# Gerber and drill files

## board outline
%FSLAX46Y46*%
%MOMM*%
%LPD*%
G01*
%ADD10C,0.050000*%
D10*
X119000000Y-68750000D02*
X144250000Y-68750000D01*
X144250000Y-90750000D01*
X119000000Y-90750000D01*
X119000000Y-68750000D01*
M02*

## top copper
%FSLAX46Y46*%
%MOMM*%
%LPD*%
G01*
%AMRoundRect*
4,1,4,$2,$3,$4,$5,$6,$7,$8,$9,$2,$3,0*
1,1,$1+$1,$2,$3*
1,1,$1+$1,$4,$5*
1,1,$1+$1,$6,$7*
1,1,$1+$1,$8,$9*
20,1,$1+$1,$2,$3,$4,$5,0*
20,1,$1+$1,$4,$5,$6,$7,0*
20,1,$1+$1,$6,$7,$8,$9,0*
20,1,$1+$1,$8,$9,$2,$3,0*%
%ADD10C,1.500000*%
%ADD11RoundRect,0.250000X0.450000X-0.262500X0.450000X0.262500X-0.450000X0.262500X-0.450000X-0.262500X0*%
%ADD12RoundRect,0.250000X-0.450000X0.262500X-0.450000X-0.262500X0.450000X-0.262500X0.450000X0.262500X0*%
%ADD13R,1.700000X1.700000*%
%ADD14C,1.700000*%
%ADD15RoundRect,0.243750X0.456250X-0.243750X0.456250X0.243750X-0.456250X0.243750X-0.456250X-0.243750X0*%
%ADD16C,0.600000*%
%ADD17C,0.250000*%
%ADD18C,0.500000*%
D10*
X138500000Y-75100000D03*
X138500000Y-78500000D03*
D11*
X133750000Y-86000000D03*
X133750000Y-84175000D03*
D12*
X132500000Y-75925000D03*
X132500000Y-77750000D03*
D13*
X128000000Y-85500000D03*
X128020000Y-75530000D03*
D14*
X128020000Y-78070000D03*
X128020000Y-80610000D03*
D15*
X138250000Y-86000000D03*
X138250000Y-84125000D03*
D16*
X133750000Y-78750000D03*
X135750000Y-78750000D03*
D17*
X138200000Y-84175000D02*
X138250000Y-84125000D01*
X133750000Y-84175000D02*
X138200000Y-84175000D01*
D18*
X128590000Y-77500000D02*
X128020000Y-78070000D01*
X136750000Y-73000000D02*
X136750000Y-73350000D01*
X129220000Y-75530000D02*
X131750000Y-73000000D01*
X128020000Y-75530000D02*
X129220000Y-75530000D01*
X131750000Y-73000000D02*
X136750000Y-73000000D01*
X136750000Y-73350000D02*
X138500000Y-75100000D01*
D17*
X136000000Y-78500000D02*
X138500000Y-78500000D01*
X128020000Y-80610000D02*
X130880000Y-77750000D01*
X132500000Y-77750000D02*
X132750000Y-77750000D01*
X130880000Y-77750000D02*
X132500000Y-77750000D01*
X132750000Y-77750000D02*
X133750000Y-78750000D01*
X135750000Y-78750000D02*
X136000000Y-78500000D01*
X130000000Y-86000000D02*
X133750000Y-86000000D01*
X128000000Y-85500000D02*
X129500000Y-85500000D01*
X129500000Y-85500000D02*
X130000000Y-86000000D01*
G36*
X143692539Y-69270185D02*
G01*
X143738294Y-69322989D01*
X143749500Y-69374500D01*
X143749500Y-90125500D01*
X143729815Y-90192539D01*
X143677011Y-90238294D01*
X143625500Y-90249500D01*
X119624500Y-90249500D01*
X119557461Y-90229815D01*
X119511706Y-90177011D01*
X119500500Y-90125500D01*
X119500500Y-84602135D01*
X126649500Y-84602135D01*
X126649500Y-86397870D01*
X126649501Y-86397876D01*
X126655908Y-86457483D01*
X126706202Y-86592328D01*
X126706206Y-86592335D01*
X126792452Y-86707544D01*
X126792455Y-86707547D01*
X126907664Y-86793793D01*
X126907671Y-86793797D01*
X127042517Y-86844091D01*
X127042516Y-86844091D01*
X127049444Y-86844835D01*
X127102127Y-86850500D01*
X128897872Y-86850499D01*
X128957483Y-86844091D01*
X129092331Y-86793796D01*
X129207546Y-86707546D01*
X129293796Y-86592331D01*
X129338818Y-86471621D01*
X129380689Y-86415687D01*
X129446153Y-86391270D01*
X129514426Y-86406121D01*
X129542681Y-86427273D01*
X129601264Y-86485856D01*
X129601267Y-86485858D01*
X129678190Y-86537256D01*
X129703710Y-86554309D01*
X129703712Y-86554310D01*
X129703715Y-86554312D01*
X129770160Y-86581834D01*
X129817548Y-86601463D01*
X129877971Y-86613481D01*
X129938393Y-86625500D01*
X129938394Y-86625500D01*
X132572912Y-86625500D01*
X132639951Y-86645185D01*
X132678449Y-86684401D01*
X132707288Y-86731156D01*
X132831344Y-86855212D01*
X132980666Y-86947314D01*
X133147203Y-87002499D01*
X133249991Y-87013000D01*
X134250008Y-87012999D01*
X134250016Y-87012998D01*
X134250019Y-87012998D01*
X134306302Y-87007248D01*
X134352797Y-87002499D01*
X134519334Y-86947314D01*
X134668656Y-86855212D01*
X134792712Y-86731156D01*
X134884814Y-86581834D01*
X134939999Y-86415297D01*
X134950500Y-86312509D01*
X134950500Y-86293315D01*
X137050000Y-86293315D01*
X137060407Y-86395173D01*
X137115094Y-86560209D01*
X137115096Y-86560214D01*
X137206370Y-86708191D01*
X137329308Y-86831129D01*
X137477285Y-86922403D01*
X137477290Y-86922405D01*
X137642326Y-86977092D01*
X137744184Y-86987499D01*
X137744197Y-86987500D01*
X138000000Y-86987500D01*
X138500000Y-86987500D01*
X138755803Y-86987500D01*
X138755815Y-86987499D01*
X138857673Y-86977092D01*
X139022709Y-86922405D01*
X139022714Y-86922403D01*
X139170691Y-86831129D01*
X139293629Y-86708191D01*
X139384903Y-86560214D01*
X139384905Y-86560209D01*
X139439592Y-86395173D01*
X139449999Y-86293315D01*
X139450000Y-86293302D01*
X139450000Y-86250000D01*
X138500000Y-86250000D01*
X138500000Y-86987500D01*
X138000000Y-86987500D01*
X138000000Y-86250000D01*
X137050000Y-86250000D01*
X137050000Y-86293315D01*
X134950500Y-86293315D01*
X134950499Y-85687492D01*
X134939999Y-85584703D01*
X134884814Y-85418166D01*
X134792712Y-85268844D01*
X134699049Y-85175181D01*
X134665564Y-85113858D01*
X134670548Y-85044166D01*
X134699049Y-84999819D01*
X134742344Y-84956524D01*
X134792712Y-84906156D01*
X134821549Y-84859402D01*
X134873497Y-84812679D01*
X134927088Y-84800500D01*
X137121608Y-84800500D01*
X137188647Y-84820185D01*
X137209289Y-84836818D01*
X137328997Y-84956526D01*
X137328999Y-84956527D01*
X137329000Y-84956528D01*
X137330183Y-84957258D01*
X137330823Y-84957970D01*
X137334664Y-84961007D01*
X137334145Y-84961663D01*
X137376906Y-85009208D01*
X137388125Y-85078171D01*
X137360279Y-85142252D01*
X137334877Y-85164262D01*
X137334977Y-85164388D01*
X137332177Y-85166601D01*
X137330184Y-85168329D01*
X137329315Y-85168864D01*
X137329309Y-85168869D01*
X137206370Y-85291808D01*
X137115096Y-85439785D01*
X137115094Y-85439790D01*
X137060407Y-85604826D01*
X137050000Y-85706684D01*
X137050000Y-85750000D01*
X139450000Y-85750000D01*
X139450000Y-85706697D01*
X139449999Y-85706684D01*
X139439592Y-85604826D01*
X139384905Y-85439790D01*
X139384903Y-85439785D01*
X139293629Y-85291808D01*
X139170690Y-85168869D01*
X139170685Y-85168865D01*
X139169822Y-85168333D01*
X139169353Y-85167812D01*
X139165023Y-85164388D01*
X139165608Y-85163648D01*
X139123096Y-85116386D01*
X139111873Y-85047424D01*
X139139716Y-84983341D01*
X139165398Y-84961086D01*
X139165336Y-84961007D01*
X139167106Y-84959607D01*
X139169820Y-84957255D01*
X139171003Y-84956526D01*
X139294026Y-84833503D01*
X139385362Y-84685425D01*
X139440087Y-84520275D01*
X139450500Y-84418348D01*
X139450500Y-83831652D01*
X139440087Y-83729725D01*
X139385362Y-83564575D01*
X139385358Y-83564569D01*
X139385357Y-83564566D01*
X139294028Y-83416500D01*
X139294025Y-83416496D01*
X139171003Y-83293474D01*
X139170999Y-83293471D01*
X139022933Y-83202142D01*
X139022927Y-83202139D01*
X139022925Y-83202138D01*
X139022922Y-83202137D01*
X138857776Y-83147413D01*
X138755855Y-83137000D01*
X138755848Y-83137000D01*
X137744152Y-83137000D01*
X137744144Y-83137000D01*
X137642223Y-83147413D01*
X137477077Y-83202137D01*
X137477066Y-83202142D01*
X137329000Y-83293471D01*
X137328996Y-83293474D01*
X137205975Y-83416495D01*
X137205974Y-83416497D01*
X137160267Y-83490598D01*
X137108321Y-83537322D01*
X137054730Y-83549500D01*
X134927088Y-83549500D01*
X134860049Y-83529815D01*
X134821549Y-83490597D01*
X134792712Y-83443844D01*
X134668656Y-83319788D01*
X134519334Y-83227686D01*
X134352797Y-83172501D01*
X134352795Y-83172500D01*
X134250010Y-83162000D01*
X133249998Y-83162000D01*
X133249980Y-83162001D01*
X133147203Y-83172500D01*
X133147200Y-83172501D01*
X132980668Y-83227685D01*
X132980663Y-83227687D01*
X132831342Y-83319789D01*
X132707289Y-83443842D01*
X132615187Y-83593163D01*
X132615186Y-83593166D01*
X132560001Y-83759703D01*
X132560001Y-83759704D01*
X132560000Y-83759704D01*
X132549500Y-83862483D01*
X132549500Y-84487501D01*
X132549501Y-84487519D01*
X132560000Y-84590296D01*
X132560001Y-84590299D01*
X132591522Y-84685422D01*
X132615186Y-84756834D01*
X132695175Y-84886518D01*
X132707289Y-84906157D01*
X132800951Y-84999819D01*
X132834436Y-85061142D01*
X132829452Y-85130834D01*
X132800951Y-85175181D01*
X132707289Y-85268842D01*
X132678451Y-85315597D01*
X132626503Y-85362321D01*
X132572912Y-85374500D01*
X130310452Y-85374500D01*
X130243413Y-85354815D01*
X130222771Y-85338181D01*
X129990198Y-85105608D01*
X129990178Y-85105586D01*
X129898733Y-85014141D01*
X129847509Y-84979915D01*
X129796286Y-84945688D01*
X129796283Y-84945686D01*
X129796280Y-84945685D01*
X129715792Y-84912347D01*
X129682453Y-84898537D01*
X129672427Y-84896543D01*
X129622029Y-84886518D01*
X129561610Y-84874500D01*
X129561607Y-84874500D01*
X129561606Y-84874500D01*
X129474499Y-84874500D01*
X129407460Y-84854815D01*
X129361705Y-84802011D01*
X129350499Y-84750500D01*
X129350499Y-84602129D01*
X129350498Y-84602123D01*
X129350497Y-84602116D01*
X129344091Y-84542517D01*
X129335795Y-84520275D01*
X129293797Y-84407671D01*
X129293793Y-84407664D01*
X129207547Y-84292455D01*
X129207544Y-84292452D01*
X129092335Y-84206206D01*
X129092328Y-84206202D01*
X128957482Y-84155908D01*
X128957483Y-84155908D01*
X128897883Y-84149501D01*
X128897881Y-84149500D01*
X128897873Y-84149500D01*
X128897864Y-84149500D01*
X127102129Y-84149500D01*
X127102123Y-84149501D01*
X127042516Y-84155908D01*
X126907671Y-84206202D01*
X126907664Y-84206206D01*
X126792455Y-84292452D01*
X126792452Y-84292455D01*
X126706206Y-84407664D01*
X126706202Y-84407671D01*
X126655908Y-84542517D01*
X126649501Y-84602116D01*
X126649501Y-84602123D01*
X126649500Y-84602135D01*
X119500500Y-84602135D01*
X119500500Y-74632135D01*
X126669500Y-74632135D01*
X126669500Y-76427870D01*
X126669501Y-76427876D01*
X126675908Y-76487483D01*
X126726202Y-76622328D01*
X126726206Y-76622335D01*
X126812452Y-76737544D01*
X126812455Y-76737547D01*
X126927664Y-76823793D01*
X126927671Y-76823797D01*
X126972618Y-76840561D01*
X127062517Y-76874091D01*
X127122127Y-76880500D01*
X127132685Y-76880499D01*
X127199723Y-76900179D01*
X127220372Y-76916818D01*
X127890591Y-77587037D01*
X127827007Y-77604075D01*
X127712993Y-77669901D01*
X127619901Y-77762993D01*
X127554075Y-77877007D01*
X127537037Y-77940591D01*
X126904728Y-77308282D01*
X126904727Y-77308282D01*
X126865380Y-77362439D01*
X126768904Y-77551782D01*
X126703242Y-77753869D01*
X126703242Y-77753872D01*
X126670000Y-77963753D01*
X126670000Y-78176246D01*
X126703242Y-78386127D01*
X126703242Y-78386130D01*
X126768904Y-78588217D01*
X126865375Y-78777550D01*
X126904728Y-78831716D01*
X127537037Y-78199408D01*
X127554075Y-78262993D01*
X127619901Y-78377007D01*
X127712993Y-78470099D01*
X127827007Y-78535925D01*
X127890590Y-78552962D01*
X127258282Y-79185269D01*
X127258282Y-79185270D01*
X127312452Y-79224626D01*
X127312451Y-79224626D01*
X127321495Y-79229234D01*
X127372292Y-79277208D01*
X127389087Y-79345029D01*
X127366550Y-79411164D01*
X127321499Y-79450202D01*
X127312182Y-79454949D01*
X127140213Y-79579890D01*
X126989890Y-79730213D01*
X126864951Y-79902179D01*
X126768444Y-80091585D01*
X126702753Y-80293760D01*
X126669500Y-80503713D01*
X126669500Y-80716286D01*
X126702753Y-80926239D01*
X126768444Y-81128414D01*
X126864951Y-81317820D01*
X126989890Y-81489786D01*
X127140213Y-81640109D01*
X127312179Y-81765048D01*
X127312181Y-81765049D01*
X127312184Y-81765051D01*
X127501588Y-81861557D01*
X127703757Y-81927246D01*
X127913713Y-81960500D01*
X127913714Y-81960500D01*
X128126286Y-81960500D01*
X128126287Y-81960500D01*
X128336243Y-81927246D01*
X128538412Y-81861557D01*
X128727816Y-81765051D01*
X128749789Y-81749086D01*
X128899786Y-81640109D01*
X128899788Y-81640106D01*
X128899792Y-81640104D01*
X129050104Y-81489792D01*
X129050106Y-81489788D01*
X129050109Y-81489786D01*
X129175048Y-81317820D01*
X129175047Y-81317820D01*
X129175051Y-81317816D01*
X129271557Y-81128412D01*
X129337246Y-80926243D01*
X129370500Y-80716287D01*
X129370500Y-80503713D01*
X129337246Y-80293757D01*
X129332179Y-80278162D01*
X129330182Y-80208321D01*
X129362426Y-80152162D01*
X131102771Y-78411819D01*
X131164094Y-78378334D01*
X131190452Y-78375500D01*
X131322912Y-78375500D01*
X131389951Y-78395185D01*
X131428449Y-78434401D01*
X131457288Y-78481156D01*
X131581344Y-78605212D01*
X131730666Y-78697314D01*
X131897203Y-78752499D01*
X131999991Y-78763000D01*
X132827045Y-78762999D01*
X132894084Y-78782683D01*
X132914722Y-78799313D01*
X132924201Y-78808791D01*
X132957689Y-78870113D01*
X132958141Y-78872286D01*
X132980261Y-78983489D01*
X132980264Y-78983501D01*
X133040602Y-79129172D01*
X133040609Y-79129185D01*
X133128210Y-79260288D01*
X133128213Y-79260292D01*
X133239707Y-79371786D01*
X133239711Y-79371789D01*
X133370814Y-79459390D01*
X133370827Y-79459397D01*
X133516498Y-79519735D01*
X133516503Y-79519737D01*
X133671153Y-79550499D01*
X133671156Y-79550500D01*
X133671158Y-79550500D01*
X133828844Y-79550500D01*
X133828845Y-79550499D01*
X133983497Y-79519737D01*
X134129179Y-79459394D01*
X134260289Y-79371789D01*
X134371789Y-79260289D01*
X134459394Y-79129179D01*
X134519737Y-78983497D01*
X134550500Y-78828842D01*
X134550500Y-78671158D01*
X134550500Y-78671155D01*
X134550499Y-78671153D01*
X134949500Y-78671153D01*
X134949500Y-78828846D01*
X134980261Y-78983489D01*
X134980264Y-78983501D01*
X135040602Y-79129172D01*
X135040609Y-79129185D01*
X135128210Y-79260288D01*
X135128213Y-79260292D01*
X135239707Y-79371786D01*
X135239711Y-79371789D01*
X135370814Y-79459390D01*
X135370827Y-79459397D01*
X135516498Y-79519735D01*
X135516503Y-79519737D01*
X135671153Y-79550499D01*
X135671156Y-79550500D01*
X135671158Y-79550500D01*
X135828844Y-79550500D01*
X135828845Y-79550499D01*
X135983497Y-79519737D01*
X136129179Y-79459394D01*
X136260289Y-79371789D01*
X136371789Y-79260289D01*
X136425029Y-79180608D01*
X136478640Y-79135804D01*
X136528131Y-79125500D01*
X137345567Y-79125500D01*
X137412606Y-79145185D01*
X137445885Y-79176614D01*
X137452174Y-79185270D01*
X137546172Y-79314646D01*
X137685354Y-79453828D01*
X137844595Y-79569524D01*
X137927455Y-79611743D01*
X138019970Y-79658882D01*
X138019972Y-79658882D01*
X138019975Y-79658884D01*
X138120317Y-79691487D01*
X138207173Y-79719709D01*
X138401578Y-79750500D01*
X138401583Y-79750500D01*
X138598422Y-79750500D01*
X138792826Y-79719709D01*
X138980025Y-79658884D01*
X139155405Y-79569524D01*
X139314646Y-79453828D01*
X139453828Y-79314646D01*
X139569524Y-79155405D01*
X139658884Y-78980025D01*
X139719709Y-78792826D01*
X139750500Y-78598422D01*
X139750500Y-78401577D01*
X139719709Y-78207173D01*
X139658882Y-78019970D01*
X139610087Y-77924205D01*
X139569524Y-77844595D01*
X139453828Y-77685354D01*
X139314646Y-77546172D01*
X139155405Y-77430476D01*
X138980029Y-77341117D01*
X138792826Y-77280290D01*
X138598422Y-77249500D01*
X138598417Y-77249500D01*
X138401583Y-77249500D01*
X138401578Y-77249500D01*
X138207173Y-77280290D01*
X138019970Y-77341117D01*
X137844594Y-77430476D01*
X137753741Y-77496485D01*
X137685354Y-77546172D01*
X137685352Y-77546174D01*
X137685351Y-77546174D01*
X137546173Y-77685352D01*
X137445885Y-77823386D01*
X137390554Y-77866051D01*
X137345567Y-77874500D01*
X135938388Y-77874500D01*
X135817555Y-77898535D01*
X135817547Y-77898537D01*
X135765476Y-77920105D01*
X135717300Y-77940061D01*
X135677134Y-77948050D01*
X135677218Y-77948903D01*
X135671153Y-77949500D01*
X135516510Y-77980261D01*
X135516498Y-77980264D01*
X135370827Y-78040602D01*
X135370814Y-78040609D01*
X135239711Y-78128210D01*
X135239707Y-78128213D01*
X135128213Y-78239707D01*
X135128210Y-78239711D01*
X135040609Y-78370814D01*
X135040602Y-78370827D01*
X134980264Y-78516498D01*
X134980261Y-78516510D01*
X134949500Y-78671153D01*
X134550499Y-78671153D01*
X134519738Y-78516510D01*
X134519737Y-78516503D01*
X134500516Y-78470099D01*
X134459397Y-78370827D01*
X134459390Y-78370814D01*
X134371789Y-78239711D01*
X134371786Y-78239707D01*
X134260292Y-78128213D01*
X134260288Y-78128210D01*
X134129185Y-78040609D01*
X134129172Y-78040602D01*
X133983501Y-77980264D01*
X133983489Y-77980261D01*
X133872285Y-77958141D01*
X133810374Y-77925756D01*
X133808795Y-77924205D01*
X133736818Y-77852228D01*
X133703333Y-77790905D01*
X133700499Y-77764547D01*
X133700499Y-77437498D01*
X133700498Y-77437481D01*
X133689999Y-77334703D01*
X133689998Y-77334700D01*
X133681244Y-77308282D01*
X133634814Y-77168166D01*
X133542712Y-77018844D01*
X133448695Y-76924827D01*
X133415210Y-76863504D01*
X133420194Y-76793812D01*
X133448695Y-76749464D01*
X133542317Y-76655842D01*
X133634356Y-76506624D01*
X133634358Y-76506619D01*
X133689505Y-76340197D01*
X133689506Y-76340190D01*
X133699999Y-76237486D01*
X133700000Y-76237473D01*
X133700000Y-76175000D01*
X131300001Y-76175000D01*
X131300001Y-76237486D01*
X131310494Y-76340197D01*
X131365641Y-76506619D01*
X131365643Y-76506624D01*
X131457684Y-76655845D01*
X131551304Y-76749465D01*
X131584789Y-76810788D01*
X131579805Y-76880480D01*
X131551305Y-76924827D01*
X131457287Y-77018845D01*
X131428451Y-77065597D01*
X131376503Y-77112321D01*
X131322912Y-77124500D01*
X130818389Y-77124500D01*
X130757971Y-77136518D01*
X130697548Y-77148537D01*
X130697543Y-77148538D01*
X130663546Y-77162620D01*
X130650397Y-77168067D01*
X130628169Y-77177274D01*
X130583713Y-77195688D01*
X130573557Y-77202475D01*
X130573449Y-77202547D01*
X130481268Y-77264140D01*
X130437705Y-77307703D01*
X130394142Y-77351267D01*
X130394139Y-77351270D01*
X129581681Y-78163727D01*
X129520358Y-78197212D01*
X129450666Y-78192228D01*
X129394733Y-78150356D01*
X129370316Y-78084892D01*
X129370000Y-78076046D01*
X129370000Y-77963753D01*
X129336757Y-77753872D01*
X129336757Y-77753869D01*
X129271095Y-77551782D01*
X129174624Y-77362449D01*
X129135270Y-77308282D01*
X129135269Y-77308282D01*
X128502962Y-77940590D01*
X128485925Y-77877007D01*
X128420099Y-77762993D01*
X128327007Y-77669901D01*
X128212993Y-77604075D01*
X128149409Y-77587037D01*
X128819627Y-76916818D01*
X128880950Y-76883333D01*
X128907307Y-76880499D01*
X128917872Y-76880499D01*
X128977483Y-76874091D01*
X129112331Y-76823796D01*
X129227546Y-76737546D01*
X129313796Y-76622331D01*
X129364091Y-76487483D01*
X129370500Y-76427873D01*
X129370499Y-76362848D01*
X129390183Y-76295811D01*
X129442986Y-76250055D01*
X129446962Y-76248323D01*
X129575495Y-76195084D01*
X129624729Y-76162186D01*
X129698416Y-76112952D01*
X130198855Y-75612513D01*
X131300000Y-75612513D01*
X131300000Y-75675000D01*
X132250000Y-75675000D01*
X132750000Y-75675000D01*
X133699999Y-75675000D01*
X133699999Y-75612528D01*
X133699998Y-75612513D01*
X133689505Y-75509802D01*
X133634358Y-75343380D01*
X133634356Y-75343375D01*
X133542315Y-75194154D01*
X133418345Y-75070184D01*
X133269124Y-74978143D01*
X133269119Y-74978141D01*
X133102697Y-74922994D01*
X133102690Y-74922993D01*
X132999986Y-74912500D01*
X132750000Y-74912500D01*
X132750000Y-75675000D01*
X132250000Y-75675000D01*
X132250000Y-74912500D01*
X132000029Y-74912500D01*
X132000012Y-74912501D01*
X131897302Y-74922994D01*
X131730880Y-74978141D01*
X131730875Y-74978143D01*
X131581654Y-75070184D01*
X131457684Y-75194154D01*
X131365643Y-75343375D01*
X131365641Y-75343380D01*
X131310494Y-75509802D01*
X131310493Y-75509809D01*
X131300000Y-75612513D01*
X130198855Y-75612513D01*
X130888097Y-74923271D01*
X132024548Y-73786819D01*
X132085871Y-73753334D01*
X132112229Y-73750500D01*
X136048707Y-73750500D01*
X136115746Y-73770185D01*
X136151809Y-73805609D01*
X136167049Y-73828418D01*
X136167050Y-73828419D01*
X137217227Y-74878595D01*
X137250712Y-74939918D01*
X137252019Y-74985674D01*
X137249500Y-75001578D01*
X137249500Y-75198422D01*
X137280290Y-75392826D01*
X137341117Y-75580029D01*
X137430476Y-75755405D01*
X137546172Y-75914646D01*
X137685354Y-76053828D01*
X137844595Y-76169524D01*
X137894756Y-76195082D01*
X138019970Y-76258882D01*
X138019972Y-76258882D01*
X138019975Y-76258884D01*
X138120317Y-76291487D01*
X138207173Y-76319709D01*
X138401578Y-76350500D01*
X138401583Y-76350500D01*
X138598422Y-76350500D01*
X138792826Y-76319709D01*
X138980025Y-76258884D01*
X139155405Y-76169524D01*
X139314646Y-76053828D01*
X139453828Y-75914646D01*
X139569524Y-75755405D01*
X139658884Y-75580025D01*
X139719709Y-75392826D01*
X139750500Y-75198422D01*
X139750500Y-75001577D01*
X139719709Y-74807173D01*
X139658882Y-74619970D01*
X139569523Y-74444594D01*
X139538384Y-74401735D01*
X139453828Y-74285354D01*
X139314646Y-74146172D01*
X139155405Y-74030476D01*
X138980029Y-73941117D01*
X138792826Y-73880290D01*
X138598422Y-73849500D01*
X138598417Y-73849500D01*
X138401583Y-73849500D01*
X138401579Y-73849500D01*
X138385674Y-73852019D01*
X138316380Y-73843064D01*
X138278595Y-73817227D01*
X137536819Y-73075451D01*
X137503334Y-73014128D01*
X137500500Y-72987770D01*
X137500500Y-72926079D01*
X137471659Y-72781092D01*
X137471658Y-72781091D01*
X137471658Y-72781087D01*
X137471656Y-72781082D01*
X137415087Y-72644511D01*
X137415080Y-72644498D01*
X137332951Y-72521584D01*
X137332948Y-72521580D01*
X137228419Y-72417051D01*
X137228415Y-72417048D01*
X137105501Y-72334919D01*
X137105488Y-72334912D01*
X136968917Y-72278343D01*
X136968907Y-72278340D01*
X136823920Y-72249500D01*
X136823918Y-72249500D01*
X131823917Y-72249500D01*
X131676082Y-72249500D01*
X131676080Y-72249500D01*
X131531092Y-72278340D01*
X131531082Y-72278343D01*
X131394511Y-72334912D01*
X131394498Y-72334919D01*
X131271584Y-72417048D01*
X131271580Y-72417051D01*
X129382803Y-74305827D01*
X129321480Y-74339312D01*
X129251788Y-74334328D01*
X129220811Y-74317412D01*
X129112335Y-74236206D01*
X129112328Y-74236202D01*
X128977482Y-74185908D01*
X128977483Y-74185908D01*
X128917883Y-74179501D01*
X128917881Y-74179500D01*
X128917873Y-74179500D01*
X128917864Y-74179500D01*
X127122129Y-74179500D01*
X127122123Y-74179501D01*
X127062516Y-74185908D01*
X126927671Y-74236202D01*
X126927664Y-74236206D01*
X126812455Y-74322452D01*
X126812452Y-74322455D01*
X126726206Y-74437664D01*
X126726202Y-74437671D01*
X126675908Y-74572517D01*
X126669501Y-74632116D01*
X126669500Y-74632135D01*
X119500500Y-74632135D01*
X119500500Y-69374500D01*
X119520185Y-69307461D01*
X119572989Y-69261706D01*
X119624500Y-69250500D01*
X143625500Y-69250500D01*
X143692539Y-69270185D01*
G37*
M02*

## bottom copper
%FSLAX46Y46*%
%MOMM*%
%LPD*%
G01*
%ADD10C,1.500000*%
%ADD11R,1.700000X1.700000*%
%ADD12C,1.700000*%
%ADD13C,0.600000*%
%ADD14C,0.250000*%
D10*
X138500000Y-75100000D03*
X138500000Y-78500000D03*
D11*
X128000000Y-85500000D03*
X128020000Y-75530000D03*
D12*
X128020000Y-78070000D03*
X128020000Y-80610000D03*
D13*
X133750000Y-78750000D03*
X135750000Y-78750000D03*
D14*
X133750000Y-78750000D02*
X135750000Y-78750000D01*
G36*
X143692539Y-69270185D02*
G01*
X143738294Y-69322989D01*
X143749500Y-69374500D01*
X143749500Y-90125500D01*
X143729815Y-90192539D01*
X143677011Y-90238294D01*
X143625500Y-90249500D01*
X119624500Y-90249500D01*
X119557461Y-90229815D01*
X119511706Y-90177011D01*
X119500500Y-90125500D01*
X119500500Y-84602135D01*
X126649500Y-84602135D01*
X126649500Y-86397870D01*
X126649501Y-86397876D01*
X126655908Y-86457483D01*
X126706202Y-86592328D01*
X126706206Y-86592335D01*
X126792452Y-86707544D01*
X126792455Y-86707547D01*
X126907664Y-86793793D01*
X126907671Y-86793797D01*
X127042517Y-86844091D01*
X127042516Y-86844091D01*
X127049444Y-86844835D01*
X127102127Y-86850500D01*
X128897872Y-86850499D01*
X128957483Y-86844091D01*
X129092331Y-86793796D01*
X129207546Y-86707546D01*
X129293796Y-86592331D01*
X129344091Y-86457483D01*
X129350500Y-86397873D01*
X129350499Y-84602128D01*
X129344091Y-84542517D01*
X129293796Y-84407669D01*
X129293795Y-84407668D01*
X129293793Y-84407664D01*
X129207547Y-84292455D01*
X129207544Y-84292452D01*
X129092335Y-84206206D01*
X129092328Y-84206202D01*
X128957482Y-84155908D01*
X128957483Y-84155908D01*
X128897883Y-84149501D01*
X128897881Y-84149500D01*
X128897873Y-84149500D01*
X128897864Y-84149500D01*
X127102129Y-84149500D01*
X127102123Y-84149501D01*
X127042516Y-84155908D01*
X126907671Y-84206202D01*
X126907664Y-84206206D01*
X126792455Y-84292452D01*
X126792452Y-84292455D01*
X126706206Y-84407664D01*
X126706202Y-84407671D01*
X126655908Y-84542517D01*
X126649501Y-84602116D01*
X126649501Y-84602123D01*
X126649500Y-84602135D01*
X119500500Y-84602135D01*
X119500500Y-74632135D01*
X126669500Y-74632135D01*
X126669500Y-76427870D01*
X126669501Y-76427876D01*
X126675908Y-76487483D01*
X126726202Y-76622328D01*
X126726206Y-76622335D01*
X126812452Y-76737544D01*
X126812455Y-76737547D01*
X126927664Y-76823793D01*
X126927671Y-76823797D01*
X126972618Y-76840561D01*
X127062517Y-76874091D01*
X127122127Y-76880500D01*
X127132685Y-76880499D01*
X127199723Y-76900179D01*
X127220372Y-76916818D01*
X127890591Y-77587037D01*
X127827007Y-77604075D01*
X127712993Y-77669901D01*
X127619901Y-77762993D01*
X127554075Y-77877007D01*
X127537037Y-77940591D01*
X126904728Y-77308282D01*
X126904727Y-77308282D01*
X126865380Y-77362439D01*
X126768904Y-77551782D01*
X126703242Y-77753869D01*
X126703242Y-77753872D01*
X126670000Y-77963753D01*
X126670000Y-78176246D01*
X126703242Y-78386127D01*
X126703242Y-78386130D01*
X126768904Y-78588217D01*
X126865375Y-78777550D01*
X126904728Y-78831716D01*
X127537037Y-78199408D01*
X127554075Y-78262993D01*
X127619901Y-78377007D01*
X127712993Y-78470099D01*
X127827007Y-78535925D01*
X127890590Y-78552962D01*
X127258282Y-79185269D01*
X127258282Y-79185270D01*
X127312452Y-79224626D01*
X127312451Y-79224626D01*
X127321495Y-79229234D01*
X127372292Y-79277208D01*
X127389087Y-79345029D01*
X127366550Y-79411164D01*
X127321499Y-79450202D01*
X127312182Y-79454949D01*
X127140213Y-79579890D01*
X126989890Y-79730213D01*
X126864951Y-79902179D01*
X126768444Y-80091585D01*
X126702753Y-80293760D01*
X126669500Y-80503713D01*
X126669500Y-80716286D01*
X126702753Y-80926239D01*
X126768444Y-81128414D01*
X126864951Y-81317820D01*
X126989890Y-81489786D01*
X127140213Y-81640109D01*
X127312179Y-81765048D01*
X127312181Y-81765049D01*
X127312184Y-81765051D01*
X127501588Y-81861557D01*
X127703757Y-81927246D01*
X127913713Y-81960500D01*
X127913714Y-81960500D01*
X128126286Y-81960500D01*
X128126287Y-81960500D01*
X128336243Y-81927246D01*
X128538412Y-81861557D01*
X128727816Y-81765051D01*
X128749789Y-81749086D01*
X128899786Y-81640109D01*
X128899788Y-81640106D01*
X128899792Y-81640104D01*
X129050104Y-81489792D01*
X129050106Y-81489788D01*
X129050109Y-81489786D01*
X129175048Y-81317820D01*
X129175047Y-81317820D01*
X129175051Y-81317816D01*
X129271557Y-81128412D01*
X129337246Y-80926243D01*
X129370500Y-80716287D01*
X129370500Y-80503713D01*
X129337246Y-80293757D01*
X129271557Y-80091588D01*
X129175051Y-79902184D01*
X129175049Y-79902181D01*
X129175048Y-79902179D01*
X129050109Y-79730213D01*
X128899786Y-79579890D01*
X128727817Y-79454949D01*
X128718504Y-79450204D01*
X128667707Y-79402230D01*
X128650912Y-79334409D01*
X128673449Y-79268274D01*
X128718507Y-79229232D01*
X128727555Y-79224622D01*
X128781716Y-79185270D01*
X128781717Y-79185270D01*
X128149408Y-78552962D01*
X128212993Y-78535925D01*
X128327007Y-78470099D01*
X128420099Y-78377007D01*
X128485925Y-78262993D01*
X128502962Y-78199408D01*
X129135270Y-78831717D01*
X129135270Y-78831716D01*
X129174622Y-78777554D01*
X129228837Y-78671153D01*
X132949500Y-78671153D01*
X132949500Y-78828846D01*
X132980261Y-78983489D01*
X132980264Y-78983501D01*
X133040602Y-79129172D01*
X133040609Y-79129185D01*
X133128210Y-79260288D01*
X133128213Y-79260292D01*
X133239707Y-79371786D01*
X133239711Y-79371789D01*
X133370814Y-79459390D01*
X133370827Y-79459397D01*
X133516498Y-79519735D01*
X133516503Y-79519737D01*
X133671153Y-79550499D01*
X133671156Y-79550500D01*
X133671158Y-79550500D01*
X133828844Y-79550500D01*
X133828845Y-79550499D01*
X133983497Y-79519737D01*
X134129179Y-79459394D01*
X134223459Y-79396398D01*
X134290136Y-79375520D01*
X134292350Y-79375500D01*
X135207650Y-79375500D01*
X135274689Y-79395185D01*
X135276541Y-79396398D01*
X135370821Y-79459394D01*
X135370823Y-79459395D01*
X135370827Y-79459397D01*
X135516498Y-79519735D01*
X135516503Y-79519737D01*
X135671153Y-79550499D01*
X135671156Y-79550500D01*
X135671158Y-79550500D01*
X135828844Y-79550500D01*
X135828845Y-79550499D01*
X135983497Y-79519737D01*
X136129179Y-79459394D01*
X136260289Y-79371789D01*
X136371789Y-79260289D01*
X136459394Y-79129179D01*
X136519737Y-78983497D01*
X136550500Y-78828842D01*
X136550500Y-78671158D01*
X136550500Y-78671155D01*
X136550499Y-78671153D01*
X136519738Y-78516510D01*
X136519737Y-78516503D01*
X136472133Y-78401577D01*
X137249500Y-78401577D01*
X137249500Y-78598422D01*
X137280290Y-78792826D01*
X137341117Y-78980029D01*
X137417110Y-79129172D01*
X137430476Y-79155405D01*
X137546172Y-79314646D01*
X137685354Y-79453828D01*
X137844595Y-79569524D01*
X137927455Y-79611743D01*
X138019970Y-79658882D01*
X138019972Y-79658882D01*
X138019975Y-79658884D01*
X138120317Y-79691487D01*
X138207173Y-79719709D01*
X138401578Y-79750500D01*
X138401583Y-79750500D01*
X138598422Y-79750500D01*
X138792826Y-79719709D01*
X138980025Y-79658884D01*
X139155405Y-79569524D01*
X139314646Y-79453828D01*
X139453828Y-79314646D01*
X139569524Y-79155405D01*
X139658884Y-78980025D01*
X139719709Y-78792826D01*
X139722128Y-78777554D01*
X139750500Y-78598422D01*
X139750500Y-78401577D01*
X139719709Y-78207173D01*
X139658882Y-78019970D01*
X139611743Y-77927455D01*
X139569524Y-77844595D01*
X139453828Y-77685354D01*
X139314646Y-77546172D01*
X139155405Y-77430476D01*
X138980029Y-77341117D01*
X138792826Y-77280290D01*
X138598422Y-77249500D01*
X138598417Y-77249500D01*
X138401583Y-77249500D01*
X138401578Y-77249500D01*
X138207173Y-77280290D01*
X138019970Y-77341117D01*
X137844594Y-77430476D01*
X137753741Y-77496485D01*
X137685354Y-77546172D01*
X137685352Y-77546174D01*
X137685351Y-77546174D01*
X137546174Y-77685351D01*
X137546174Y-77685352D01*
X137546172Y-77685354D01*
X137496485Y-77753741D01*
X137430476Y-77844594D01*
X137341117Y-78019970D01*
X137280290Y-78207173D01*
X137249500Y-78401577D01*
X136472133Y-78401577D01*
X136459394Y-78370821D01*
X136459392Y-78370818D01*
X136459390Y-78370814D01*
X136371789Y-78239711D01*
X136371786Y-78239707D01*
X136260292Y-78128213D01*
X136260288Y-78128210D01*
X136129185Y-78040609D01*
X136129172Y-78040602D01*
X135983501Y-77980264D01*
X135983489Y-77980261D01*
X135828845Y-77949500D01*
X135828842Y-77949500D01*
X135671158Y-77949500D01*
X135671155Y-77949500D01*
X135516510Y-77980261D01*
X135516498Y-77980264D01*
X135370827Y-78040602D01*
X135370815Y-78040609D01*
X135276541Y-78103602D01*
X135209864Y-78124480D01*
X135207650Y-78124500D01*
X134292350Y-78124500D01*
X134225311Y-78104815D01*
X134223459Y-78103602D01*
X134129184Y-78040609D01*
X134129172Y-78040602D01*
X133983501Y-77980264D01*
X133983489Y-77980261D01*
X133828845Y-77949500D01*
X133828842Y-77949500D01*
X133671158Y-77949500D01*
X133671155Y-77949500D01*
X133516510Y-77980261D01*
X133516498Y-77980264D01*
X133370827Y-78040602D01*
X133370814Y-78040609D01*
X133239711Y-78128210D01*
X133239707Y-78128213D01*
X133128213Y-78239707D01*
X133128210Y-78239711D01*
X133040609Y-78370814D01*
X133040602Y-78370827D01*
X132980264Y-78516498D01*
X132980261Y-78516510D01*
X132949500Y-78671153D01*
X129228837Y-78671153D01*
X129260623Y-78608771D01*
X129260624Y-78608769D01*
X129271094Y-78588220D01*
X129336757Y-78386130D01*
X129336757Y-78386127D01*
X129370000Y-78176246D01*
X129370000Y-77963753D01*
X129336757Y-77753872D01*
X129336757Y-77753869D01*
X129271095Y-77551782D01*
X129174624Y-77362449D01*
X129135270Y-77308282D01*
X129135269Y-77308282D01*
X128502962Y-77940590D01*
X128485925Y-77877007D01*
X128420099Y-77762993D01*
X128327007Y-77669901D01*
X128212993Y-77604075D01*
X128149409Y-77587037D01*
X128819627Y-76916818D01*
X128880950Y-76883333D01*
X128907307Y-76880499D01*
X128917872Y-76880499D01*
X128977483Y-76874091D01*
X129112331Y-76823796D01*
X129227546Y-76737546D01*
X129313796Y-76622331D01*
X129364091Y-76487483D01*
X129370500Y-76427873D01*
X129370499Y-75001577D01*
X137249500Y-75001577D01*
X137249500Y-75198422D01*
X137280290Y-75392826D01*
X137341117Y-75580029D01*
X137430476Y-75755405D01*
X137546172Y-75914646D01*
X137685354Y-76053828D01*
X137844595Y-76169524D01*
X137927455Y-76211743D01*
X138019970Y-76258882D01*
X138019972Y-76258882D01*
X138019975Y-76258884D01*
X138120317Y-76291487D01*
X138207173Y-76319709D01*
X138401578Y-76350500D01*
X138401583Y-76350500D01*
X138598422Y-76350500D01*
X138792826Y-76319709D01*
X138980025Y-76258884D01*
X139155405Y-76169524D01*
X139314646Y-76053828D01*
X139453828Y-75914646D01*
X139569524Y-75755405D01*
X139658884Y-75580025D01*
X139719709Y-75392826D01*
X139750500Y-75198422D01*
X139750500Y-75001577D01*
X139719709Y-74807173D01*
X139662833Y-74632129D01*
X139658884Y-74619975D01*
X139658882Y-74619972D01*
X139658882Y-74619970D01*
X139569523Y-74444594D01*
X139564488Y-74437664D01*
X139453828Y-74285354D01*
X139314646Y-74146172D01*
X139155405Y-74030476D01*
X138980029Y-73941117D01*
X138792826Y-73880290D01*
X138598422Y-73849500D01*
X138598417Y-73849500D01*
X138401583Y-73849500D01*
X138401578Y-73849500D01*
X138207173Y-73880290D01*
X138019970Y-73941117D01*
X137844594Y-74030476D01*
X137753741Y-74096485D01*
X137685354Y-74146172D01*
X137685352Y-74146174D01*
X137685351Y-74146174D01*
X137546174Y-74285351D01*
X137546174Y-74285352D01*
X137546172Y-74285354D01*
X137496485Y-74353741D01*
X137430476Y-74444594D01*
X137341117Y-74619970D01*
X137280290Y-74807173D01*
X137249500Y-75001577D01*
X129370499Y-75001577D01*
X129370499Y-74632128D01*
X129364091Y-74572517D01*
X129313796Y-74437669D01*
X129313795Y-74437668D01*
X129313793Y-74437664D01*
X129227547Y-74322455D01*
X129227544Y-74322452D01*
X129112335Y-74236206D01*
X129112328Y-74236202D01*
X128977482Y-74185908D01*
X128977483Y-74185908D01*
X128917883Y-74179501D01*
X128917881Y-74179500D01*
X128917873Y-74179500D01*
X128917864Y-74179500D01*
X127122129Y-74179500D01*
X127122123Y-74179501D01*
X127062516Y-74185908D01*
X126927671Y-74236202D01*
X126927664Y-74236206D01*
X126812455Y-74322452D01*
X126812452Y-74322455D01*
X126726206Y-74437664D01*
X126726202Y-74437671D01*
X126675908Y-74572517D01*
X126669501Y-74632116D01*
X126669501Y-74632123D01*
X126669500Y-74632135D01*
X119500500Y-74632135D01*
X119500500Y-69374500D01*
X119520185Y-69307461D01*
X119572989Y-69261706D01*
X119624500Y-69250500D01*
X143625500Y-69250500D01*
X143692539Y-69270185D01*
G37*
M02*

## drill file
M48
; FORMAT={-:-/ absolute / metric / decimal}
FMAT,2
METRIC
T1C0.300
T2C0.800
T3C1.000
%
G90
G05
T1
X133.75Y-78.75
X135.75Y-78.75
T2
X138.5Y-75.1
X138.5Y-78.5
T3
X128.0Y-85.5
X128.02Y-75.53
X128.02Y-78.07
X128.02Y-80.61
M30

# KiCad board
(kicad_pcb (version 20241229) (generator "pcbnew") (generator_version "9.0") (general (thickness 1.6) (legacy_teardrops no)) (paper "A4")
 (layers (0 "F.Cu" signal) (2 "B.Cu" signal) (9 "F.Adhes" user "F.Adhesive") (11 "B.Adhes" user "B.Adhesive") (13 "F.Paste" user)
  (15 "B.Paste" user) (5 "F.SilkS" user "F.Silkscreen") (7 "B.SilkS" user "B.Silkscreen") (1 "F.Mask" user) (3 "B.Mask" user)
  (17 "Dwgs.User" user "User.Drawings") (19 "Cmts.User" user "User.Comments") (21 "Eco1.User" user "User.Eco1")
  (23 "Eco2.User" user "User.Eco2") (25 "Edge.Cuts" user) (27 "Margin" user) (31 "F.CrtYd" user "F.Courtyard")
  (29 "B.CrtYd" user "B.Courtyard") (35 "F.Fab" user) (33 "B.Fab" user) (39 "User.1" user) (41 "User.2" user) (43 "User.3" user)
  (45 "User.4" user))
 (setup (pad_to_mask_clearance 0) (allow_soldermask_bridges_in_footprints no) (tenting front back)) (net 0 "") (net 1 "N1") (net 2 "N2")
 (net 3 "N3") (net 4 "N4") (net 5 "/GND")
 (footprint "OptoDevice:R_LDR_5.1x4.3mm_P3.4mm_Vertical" (layer "F.Cu") (at 138.5 75.1 -90)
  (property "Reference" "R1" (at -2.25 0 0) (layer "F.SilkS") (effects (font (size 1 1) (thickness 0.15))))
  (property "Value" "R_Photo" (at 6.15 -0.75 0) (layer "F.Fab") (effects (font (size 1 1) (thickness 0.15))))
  (pad "1" thru_hole circle (at 0 0 270) (size 1.5 1.5) (drill 0.8) (layers "*.Cu" "*.Mask") (remove_unused_layers no) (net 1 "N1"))
  (pad "2" thru_hole circle (at 3.4 0 270) (size 1.5 1.5) (drill 0.8) (layers "*.Cu" "*.Mask") (remove_unused_layers no) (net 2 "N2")))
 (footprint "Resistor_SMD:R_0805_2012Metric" (layer "F.Cu") (at 133.75 85.0875 90)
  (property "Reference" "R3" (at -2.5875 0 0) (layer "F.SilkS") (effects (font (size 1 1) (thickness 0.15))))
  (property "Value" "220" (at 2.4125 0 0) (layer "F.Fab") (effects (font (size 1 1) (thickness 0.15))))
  (pad "1" smd roundrect (at -0.9125 0 90) (size 1.025 1.4) (layers "F.Cu" "F.Mask" "F.Paste") (roundrect_rratio 0.243902) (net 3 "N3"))
  (pad "2" smd roundrect (at 0.9125 0 90) (size 1.025 1.4) (layers "F.Cu" "F.Mask" "F.Paste") (roundrect_rratio 0.243902) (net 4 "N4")))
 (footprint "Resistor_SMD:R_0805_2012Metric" (layer "F.Cu") (at 132.5 76.8375 -90)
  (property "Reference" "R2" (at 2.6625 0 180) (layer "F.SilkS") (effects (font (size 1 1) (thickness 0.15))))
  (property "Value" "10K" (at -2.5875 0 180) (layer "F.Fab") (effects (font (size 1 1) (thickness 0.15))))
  (pad "1" smd roundrect (at -0.9125 0 270) (size 1.025 1.4) (layers "F.Cu" "F.Mask" "F.Paste") (roundrect_rratio 0.243902) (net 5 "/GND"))
  (pad "2" smd roundrect (at 0.9125 0 270) (size 1.025 1.4) (layers "F.Cu" "F.Mask" "F.Paste") (roundrect_rratio 0.243902) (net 2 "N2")))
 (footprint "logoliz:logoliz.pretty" (layer "F.Cu") (at 122.5 72)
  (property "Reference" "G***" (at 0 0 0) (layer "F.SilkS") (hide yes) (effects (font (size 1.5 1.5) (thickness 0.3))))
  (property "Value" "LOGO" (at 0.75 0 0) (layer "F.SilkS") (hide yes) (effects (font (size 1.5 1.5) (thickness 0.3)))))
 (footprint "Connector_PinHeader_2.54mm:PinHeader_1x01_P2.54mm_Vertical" (layer "F.Cu") (at 128 85.5)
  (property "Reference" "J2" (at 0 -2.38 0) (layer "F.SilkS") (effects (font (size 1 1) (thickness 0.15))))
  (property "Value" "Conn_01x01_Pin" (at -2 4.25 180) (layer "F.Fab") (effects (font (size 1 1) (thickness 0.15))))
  (pad "1" thru_hole rect (at 0 0) (size 1.7 1.7) (drill 1) (layers "*.Cu" "*.Mask") (remove_unused_layers no) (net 3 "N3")))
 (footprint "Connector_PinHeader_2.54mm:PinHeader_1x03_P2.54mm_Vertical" (layer "F.Cu") (at 128.02 75.53)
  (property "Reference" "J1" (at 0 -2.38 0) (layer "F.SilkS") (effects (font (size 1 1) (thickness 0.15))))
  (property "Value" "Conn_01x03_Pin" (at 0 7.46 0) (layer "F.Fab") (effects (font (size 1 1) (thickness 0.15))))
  (pad "1" thru_hole rect (at 0 0) (size 1.7 1.7) (drill 1) (layers "*.Cu" "*.Mask") (remove_unused_layers no) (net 1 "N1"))
  (pad "2" thru_hole circle (at 0 2.54) (size 1.7 1.7) (drill 1) (layers "*.Cu" "*.Mask") (remove_unused_layers no) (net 5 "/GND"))
  (pad "3" thru_hole circle (at 0 5.08) (size 1.7 1.7) (drill 1) (layers "*.Cu" "*.Mask") (remove_unused_layers no) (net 2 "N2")))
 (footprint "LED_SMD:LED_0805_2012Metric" (layer "F.Cu") (at 138.25 85.0625 90)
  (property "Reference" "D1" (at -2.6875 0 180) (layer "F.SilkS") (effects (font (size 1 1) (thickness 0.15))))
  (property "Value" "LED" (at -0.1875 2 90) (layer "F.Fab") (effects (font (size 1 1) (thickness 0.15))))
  (pad "1" smd roundrect (at -0.9375 0 90) (size 0.975 1.4) (layers "F.Cu" "F.Mask" "F.Paste") (roundrect_rratio 0.25) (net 5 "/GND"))
  (pad "2" smd roundrect (at 0.9375 0 90) (size 0.975 1.4) (layers "F.Cu" "F.Mask" "F.Paste") (roundrect_rratio 0.25) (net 4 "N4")))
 (gr_rect (start 119 68.75) (end 144.25 90.75) (stroke (width 0.05) (type default)) (fill no) (layer "Edge.Cuts"))
 (segment (start 138.2 84.175) (end 138.25 84.125) (width 0.25) (layer "F.Cu") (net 4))
 (segment (start 133.75 84.175) (end 138.2 84.175) (width 0.25) (layer "F.Cu") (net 4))
 (segment (start 128.59 77.5) (end 128.02 78.07) (width 0.5) (layer "F.Cu") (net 5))
 (segment (start 136.75 73) (end 136.75 73.35) (width 0.5) (layer "F.Cu") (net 1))
 (segment (start 129.22 75.53) (end 131.75 73) (width 0.5) (layer "F.Cu") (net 1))
 (segment (start 128.02 75.53) (end 129.22 75.53) (width 0.5) (layer "F.Cu") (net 1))
 (segment (start 131.75 73) (end 136.75 73) (width 0.5) (layer "F.Cu") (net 1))
 (segment (start 136.75 73.35) (end 138.5 75.1) (width 0.5) (layer "F.Cu") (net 1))
 (segment (start 136 78.5) (end 138.5 78.5) (width 0.25) (layer "F.Cu") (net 2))
 (segment (start 128.02 80.61) (end 130.88 77.75) (width 0.25) (layer "F.Cu") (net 2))
 (segment (start 132.5 77.75) (end 132.75 77.75) (width 0.25) (layer "F.Cu") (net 2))
 (segment (start 130.88 77.75) (end 132.5 77.75) (width 0.25) (layer "F.Cu") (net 2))
 (segment (start 132.75 77.75) (end 133.75 78.75) (width 0.25) (layer "F.Cu") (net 2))
 (segment (start 135.75 78.75) (end 136 78.5) (width 0.25) (layer "F.Cu") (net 2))
 (via (at 133.75 78.75) (size 0.6) (drill 0.3) (layers "F.Cu" "B.Cu") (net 2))
 (via (at 135.75 78.75) (size 0.6) (drill 0.3) (layers "F.Cu" "B.Cu") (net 2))
 (segment (start 133.75 78.75) (end 135.75 78.75) (width 0.25) (layer "B.Cu") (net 2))
 (segment (start 130 86) (end 133.75 86) (width 0.25) (layer "F.Cu") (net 3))
 (segment (start 128 85.5) (end 129.5 85.5) (width 0.25) (layer "F.Cu") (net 3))
 (segment (start 129.5 85.5) (end 130 86) (width 0.25) (layer "F.Cu") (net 3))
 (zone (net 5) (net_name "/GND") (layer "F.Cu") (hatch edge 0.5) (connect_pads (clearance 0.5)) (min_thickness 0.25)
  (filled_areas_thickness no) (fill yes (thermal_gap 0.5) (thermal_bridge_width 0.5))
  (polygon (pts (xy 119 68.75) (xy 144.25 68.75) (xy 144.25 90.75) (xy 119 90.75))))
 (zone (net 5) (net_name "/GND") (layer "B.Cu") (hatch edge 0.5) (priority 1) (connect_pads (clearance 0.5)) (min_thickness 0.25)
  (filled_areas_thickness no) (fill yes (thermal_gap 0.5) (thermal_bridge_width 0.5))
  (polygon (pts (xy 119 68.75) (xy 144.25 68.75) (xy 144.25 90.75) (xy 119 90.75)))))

